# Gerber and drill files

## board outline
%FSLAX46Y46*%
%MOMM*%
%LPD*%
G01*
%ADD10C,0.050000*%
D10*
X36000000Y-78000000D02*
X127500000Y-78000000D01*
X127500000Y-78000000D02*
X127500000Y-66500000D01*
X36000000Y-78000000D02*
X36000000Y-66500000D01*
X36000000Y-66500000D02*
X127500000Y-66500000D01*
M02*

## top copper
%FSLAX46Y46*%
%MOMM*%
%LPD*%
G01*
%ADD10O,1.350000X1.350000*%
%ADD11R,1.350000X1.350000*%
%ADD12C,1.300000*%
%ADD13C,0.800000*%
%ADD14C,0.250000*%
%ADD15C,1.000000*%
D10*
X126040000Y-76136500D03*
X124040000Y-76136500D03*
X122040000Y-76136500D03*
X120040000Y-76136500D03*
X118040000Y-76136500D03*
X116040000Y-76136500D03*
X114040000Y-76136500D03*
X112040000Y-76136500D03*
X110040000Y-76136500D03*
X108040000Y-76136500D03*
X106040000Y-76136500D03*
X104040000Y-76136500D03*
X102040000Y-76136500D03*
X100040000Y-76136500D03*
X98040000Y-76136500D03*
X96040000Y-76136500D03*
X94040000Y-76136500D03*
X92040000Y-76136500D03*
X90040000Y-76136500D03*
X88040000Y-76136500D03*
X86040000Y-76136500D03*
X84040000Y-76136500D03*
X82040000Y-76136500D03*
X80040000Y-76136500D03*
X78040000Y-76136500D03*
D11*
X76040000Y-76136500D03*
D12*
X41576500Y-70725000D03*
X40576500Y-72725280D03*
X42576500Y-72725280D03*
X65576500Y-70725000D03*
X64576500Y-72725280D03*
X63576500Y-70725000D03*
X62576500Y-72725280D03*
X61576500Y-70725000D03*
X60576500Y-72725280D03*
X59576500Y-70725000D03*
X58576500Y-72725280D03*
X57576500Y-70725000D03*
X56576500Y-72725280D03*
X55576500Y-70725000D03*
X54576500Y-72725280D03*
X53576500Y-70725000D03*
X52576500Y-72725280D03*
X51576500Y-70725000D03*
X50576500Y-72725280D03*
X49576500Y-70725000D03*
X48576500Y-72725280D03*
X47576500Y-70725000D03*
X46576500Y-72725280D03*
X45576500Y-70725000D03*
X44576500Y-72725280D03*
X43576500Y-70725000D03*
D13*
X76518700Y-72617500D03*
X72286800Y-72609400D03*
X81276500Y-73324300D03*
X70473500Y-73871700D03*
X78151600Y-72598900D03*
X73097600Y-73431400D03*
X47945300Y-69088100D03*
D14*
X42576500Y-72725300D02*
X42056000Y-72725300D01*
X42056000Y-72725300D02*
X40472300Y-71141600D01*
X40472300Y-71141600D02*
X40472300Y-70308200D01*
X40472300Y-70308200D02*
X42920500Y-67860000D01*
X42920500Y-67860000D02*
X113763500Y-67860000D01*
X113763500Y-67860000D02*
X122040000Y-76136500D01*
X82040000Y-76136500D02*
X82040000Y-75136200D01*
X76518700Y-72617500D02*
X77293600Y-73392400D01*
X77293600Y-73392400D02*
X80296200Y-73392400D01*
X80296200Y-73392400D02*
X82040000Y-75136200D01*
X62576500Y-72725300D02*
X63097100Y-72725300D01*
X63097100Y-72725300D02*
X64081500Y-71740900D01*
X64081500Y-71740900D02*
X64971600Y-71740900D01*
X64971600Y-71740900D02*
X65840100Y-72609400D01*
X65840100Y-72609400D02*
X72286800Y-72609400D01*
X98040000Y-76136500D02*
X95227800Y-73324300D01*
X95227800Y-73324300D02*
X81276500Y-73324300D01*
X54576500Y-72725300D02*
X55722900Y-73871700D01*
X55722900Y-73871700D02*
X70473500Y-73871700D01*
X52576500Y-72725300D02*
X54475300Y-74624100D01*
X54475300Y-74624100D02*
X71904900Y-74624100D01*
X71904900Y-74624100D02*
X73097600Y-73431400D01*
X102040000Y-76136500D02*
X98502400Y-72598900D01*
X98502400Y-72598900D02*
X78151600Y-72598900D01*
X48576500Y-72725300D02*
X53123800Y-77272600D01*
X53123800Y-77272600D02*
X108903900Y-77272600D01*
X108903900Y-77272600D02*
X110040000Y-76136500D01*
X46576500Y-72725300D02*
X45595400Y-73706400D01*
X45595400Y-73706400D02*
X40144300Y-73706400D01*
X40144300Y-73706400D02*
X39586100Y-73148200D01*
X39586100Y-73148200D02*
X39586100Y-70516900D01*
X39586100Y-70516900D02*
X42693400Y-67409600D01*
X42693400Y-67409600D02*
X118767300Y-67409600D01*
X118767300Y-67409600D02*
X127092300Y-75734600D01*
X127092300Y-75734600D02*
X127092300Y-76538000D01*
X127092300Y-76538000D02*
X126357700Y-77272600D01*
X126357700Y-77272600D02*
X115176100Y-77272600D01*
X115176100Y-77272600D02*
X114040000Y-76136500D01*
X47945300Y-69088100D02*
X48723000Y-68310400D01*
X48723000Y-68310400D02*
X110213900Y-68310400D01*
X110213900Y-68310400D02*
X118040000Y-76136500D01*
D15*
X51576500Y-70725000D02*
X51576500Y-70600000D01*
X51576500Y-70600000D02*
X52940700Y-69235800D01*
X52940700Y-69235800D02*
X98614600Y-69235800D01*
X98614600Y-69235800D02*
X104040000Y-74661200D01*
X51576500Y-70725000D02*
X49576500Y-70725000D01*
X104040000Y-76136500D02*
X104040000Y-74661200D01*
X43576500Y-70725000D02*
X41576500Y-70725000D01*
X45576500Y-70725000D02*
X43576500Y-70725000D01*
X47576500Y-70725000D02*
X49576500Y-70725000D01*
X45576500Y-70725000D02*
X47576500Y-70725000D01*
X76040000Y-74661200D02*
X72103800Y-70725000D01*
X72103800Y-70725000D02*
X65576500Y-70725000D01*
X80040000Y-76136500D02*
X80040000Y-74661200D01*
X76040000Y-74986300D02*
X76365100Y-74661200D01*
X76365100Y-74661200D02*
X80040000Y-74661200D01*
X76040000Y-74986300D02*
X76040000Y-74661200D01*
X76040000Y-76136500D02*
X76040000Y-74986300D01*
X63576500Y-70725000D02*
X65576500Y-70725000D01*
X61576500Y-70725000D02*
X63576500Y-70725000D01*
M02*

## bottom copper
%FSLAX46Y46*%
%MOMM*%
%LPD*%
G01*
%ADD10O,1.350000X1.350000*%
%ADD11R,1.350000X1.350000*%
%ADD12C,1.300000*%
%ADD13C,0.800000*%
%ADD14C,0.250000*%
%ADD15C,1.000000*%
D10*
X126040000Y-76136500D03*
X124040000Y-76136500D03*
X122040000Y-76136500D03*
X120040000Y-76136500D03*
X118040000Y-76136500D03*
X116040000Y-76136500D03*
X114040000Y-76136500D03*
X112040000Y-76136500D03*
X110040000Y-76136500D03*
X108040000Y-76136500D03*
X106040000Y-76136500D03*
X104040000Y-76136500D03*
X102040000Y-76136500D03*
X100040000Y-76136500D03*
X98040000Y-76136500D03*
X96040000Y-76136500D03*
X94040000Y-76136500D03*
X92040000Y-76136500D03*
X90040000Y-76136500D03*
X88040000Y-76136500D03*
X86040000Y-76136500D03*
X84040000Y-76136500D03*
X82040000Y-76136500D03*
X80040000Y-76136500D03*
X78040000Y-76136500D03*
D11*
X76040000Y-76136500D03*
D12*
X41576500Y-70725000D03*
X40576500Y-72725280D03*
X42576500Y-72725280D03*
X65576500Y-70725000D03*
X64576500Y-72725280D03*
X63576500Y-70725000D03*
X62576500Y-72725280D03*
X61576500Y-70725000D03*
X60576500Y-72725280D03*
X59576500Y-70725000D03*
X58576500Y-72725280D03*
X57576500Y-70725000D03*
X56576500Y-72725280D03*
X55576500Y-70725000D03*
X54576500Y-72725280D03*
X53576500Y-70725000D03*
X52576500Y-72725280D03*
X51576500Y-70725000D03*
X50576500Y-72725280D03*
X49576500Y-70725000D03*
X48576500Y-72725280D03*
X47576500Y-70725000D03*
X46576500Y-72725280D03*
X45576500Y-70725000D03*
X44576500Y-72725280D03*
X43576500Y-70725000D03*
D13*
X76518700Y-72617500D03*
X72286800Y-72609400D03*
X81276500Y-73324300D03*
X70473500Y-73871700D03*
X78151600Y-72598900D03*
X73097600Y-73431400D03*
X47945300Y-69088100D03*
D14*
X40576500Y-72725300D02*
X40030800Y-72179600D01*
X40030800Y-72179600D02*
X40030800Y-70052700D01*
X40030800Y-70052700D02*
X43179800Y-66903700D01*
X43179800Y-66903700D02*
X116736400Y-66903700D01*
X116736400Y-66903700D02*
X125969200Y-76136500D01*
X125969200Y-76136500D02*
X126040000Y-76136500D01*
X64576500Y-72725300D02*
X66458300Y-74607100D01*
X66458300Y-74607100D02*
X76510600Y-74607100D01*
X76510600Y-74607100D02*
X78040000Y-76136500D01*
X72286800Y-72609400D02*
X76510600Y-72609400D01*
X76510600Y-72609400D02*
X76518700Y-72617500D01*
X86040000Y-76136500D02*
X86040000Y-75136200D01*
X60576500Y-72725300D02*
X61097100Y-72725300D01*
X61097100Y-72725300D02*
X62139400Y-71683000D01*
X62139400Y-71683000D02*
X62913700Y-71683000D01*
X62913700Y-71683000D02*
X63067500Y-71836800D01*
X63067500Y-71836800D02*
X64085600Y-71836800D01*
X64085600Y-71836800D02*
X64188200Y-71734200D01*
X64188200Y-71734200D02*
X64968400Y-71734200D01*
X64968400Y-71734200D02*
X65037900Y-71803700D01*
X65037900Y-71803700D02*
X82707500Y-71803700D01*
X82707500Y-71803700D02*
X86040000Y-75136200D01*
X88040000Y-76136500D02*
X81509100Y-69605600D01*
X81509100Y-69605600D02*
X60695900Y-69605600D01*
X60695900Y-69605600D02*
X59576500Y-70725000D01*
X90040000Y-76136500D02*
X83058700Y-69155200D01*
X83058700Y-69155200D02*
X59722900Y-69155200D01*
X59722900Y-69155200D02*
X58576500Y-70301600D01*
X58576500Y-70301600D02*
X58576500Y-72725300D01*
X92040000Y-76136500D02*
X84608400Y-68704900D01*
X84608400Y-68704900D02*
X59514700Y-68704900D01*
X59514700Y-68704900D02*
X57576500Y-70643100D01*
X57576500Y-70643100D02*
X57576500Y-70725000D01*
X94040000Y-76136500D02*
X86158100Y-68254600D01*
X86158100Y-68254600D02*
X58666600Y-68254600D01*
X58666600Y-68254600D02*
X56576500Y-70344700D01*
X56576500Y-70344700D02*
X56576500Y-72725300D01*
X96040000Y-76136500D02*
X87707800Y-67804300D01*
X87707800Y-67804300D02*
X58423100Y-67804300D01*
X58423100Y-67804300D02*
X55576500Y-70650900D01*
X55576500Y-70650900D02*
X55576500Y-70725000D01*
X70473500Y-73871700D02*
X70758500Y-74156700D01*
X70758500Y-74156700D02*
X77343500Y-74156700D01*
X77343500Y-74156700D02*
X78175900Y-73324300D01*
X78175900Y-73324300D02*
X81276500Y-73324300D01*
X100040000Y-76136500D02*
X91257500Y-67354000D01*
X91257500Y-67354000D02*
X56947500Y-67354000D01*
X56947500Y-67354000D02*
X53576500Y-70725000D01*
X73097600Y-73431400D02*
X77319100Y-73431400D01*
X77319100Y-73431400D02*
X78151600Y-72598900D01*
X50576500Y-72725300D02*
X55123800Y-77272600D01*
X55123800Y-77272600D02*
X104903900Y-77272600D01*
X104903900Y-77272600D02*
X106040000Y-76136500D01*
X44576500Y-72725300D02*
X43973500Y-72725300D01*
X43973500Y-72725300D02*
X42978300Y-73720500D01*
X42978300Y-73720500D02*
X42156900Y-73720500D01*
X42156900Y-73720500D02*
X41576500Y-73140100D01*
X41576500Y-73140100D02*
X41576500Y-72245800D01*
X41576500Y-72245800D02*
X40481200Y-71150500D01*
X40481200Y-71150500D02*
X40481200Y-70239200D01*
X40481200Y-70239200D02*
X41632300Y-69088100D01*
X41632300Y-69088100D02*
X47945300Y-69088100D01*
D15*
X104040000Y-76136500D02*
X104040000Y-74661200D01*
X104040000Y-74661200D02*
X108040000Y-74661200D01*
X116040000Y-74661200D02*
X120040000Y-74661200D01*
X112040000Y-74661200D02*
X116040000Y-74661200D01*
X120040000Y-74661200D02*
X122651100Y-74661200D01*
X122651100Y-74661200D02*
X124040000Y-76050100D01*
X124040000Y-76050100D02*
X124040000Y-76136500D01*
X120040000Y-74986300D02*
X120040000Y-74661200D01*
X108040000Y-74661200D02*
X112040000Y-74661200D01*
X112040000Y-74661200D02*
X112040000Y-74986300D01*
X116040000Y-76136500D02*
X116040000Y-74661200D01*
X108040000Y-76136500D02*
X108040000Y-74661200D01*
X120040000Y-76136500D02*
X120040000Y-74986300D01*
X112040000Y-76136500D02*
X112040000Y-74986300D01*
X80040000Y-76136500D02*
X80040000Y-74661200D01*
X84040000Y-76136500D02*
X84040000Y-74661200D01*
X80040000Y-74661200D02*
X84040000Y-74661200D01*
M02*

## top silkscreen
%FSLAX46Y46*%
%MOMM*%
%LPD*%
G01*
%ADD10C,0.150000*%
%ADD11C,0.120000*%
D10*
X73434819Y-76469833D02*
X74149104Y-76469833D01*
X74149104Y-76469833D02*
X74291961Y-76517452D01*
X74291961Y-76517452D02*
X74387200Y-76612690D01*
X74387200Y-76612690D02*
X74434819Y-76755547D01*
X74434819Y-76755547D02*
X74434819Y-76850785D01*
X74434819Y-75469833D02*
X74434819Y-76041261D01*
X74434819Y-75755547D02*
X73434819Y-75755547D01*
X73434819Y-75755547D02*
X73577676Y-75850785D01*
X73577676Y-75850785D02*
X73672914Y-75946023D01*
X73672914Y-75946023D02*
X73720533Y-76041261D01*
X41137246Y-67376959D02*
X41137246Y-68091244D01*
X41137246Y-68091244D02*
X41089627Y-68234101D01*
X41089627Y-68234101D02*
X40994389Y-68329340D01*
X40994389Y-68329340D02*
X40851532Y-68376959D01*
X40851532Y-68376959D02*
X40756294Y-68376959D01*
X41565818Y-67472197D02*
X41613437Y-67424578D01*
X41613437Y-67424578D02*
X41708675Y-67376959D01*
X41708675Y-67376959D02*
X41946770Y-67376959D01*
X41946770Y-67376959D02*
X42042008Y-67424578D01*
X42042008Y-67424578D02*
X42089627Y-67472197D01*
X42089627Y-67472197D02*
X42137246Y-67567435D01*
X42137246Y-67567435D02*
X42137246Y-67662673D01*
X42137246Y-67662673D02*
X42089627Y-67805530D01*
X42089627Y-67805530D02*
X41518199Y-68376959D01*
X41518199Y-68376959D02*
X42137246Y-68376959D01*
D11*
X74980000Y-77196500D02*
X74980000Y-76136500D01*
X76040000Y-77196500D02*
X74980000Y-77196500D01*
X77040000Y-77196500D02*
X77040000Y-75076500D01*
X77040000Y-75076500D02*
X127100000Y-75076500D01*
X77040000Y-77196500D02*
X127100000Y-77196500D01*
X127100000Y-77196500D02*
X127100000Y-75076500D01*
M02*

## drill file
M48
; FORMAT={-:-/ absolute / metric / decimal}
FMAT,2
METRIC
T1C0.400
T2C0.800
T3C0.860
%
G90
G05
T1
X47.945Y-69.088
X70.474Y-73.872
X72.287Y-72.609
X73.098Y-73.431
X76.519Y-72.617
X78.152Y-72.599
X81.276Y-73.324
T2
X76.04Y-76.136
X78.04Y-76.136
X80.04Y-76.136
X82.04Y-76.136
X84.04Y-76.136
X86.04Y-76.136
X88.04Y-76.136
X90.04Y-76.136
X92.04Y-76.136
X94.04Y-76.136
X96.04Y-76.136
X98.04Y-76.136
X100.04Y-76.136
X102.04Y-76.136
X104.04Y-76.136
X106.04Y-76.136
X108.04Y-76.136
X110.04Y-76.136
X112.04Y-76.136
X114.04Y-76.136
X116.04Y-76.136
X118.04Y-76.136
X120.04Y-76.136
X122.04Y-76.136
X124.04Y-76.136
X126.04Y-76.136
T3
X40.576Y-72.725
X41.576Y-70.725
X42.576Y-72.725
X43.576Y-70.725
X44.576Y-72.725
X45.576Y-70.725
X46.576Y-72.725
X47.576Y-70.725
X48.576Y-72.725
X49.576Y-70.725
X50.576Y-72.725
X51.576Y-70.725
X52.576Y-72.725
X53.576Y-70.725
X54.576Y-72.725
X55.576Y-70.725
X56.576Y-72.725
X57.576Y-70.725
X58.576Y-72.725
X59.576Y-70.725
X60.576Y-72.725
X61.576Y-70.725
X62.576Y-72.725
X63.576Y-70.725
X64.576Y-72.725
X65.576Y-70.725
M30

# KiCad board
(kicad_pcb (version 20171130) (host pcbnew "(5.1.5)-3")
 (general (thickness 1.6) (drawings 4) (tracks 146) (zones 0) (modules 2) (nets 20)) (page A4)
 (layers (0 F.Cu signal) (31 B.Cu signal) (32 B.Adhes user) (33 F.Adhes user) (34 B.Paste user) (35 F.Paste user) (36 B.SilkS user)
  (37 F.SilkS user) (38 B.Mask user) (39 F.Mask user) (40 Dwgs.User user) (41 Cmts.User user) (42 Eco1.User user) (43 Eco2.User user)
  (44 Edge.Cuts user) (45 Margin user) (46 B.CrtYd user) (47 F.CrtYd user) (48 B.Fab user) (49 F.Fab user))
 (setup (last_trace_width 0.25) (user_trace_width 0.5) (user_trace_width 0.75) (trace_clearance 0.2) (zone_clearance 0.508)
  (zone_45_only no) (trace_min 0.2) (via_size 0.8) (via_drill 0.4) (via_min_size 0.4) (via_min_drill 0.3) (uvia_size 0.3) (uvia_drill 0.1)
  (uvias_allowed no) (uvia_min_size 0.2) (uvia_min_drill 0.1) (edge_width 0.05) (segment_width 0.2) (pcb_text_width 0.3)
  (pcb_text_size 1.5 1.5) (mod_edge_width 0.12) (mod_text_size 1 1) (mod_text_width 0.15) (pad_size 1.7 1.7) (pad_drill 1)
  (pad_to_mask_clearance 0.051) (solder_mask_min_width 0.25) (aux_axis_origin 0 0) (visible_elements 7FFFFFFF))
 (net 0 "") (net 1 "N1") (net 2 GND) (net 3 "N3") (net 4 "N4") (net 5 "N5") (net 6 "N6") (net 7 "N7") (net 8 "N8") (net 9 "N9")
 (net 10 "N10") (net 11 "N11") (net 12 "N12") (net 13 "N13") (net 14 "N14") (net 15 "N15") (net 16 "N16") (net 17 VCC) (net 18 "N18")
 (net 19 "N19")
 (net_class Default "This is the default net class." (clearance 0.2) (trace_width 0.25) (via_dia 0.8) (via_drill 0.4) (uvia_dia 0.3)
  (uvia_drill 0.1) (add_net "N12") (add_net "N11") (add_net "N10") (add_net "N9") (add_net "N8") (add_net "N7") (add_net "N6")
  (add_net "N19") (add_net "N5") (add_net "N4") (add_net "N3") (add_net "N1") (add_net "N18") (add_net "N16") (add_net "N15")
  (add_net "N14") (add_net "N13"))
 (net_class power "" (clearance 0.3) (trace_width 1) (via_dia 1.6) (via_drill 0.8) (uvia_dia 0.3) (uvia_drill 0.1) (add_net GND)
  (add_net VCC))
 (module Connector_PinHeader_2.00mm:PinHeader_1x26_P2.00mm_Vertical (layer F.Cu) (at 76.04 76.1365 90)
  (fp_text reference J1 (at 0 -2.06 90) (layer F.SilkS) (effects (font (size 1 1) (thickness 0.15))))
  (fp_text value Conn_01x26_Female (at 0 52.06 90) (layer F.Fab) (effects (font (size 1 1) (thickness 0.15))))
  (fp_line (start -1.06 -1.06) (end 0 -1.06) (layer F.SilkS) (width 0.12))
  (fp_line (start -1.06 0) (end -1.06 -1.06) (layer F.SilkS) (width 0.12))
  (fp_line (start -1.06 1) (end 1.06 1) (layer F.SilkS) (width 0.12))
  (fp_line (start 1.06 1) (end 1.06 51.06) (layer F.SilkS) (width 0.12))
  (fp_line (start -1.06 1) (end -1.06 51.06) (layer F.SilkS) (width 0.12))
  (fp_line (start -1.06 51.06) (end 1.06 51.06) (layer F.SilkS) (width 0.12))
  (pad 26 thru_hole oval (at 0 50 90) (size 1.35 1.35) (drill 0.8) (layers *.Cu *.Mask) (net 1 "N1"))
  (pad 25 thru_hole oval (at 0 48 90) (size 1.35 1.35) (drill 0.8) (layers *.Cu *.Mask) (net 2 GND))
  (pad 24 thru_hole oval (at 0 46 90) (size 1.35 1.35) (drill 0.8) (layers *.Cu *.Mask) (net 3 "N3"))
  (pad 23 thru_hole oval (at 0 44 90) (size 1.35 1.35) (drill 0.8) (layers *.Cu *.Mask) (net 2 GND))
  (pad 22 thru_hole oval (at 0 42 90) (size 1.35 1.35) (drill 0.8) (layers *.Cu *.Mask) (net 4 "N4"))
  (pad 21 thru_hole oval (at 0 40 90) (size 1.35 1.35) (drill 0.8) (layers *.Cu *.Mask) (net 2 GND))
  (pad 20 thru_hole oval (at 0 38 90) (size 1.35 1.35) (drill 0.8) (layers *.Cu *.Mask) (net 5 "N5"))
  (pad 19 thru_hole oval (at 0 36 90) (size 1.35 1.35) (drill 0.8) (layers *.Cu *.Mask) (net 2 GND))
  (pad 18 thru_hole oval (at 0 34 90) (size 1.35 1.35) (drill 0.8) (layers *.Cu *.Mask) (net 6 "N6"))
  (pad 17 thru_hole oval (at 0 32 90) (size 1.35 1.35) (drill 0.8) (layers *.Cu *.Mask) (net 2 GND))
  (pad 16 thru_hole oval (at 0 30 90) (size 1.35 1.35) (drill 0.8) (layers *.Cu *.Mask) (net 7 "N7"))
  (pad 15 thru_hole oval (at 0 28 90) (size 1.35 1.35) (drill 0.8) (layers *.Cu *.Mask) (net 2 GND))
  (pad 14 thru_hole oval (at 0 26 90) (size 1.35 1.35) (drill 0.8) (layers *.Cu *.Mask) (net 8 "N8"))
  (pad 13 thru_hole oval (at 0 24 90) (size 1.35 1.35) (drill 0.8) (layers *.Cu *.Mask) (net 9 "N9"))
  (pad 12 thru_hole oval (at 0 22 90) (size 1.35 1.35) (drill 0.8) (layers *.Cu *.Mask) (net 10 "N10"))
  (pad 11 thru_hole oval (at 0 20 90) (size 1.35 1.35) (drill 0.8) (layers *.Cu *.Mask) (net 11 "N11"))
  (pad 10 thru_hole oval (at 0 18 90) (size 1.35 1.35) (drill 0.8) (layers *.Cu *.Mask) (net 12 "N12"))
  (pad 9 thru_hole oval (at 0 16 90) (size 1.35 1.35) (drill 0.8) (layers *.Cu *.Mask) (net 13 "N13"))
  (pad 8 thru_hole oval (at 0 14 90) (size 1.35 1.35) (drill 0.8) (layers *.Cu *.Mask) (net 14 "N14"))
  (pad 7 thru_hole oval (at 0 12 90) (size 1.35 1.35) (drill 0.8) (layers *.Cu *.Mask) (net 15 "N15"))
  (pad 6 thru_hole oval (at 0 10 90) (size 1.35 1.35) (drill 0.8) (layers *.Cu *.Mask) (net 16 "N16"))
  (pad 5 thru_hole oval (at 0 8 90) (size 1.35 1.35) (drill 0.8) (layers *.Cu *.Mask) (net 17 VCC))
  (pad 4 thru_hole oval (at 0 6 90) (size 1.35 1.35) (drill 0.8) (layers *.Cu *.Mask) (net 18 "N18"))
  (pad 3 thru_hole oval (at 0 4 90) (size 1.35 1.35) (drill 0.8) (layers *.Cu *.Mask) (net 17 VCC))
  (pad 2 thru_hole oval (at 0 2 90) (size 1.35 1.35) (drill 0.8) (layers *.Cu *.Mask) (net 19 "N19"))
  (pad 1 thru_hole rect (at 0 0 90) (size 1.35 1.35) (drill 0.8) (layers *.Cu *.Mask) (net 17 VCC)))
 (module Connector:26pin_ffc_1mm (layer F.Cu) (at 40.5765 75.438)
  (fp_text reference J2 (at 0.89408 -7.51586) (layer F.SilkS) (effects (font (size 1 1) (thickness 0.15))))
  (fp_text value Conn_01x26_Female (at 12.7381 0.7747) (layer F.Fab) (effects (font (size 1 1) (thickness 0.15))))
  (pad 25 thru_hole circle (at 1 -4.713) (size 1.3 1.3) (drill 0.86) (layers *.Cu *.Mask) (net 2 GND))
  (pad 26 thru_hole circle (at 0 -2.71272) (size 1.3 1.3) (drill 0.86) (layers *.Cu *.Mask) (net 1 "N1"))
  (pad 24 thru_hole circle (at 2 -2.71272) (size 1.3 1.3) (drill 0.86) (layers *.Cu *.Mask) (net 3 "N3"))
  (pad 1 thru_hole circle (at 25 -4.713) (size 1.3 1.3) (drill 0.86) (layers *.Cu *.Mask) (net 17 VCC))
  (pad 2 thru_hole circle (at 24 -2.71272) (size 1.3 1.3) (drill 0.86) (layers *.Cu *.Mask) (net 19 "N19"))
  (pad 3 thru_hole circle (at 23 -4.713) (size 1.3 1.3) (drill 0.86) (layers *.Cu *.Mask) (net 17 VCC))
  (pad 4 thru_hole circle (at 22 -2.71272) (size 1.3 1.3) (drill 0.86) (layers *.Cu *.Mask) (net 18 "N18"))
  (pad 5 thru_hole circle (at 21 -4.713) (size 1.3 1.3) (drill 0.86) (layers *.Cu *.Mask) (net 17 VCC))
  (pad 6 thru_hole circle (at 20 -2.71272) (size 1.3 1.3) (drill 0.86) (layers *.Cu *.Mask) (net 16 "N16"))
  (pad 7 thru_hole circle (at 19 -4.713) (size 1.3 1.3) (drill 0.86) (layers *.Cu *.Mask) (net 15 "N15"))
  (pad 8 thru_hole circle (at 18 -2.71272) (size 1.3 1.3) (drill 0.86) (layers *.Cu *.Mask) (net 14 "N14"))
  (pad 9 thru_hole circle (at 17 -4.713) (size 1.3 1.3) (drill 0.86) (layers *.Cu *.Mask) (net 13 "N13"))
  (pad 10 thru_hole circle (at 16 -2.71272) (size 1.3 1.3) (drill 0.86) (layers *.Cu *.Mask) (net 12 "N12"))
  (pad 11 thru_hole circle (at 15 -4.713) (size 1.3 1.3) (drill 0.86) (layers *.Cu *.Mask) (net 11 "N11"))
  (pad 12 thru_hole circle (at 14 -2.71272) (size 1.3 1.3) (drill 0.86) (layers *.Cu *.Mask) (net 10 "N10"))
  (pad 13 thru_hole circle (at 13 -4.713) (size 1.3 1.3) (drill 0.86) (layers *.Cu *.Mask) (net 9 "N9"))
  (pad 14 thru_hole circle (at 12 -2.71272) (size 1.3 1.3) (drill 0.86) (layers *.Cu *.Mask) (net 8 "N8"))
  (pad 15 thru_hole circle (at 11 -4.713) (size 1.3 1.3) (drill 0.86) (layers *.Cu *.Mask) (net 2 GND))
  (pad 16 thru_hole circle (at 10 -2.71272) (size 1.3 1.3) (drill 0.86) (layers *.Cu *.Mask) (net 7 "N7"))
  (pad 17 thru_hole circle (at 9 -4.713) (size 1.3 1.3) (drill 0.86) (layers *.Cu *.Mask) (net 2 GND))
  (pad 18 thru_hole circle (at 8 -2.71272) (size 1.3 1.3) (drill 0.86) (layers *.Cu *.Mask) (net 6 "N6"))
  (pad 19 thru_hole circle (at 7 -4.713) (size 1.3 1.3) (drill 0.86) (layers *.Cu *.Mask) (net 2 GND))
  (pad 20 thru_hole circle (at 6 -2.71272) (size 1.3 1.3) (drill 0.86) (layers *.Cu *.Mask) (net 5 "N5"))
  (pad 21 thru_hole circle (at 5 -4.713) (size 1.3 1.3) (drill 0.86) (layers *.Cu *.Mask) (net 2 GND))
  (pad 22 thru_hole circle (at 4 -2.71272) (size 1.3 1.3) (drill 0.86) (layers *.Cu *.Mask) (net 4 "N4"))
  (pad 23 thru_hole circle (at 3 -4.713) (size 1.3 1.3) (drill 0.86) (layers *.Cu *.Mask) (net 2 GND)))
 (gr_line (start 36 78) (end 127.5 78) (layer Edge.Cuts) (width 0.05))
 (gr_line (start 127.5 78) (end 127.5 66.5) (layer Edge.Cuts) (width 0.05))
 (gr_line (start 36 78) (end 36 66.5) (layer Edge.Cuts) (width 0.05))
 (gr_line (start 36 66.5) (end 127.5 66.5) (layer Edge.Cuts) (width 0.05))
 (segment (start 40.5765 72.7253) (end 40.0308 72.1796) (width 0.25) (layer B.Cu) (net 1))
 (segment (start 40.0308 72.1796) (end 40.0308 70.0527) (width 0.25) (layer B.Cu) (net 1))
 (segment (start 40.0308 70.0527) (end 43.1798 66.9037) (width 0.25) (layer B.Cu) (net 1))
 (segment (start 43.1798 66.9037) (end 116.7364 66.9037) (width 0.25) (layer B.Cu) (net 1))
 (segment (start 116.7364 66.9037) (end 125.9692 76.1365) (width 0.25) (layer B.Cu) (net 1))
 (segment (start 125.9692 76.1365) (end 126.04 76.1365) (width 0.25) (layer B.Cu) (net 1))
 (segment (start 42.5765 72.7253) (end 42.056 72.7253) (width 0.25) (layer F.Cu) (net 3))
 (segment (start 42.056 72.7253) (end 40.4723 71.1416) (width 0.25) (layer F.Cu) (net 3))
 (segment (start 40.4723 71.1416) (end 40.4723 70.3082) (width 0.25) (layer F.Cu) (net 3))
 (segment (start 40.4723 70.3082) (end 42.9205 67.86) (width 0.25) (layer F.Cu) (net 3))
 (segment (start 42.9205 67.86) (end 113.7635 67.86) (width 0.25) (layer F.Cu) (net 3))
 (segment (start 113.7635 67.86) (end 122.04 76.1365) (width 0.25) (layer F.Cu) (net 3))
 (segment (start 64.5765 72.7253) (end 66.4583 74.6071) (width 0.25) (layer B.Cu) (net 19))
 (segment (start 66.4583 74.6071) (end 76.5106 74.6071) (width 0.25) (layer B.Cu) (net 19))
 (segment (start 76.5106 74.6071) (end 78.04 76.1365) (width 0.25) (layer B.Cu) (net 19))
 (segment (start 82.04 76.1365) (end 82.04 75.1362) (width 0.25) (layer F.Cu) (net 18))
 (segment (start 76.5187 72.6175) (end 77.2936 73.3924) (width 0.25) (layer F.Cu) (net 18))
 (segment (start 77.2936 73.3924) (end 80.2962 73.3924) (width 0.25) (layer F.Cu) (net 18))
 (segment (start 80.2962 73.3924) (end 82.04 75.1362) (width 0.25) (layer F.Cu) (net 18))
 (segment (start 72.2868 72.6094) (end 76.5106 72.6094) (width 0.25) (layer B.Cu) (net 18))
 (segment (start 76.5106 72.6094) (end 76.5187 72.6175) (width 0.25) (layer B.Cu) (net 18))
 (segment (start 62.5765 72.7253) (end 63.0971 72.7253) (width 0.25) (layer F.Cu) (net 18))
 (segment (start 63.0971 72.7253) (end 64.0815 71.7409) (width 0.25) (layer F.Cu) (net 18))
 (segment (start 64.0815 71.7409) (end 64.9716 71.7409) (width 0.25) (layer F.Cu) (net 18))
 (segment (start 64.9716 71.7409) (end 65.8401 72.6094) (width 0.25) (layer F.Cu) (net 18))
 (segment (start 65.8401 72.6094) (end 72.2868 72.6094) (width 0.25) (layer F.Cu) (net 18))
 (via (at 76.5187 72.6175) (size 0.8) (layers F.Cu B.Cu) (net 18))
 (via (at 72.2868 72.6094) (size 0.8) (layers F.Cu B.Cu) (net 18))
 (segment (start 86.04 76.1365) (end 86.04 75.1362) (width 0.25) (layer B.Cu) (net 16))
 (segment (start 60.5765 72.7253) (end 61.0971 72.7253) (width 0.25) (layer B.Cu) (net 16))
 (segment (start 61.0971 72.7253) (end 62.1394 71.683) (width 0.25) (layer B.Cu) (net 16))
 (segment (start 62.1394 71.683) (end 62.9137 71.683) (width 0.25) (layer B.Cu) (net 16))
 (segment (start 62.9137 71.683) (end 63.0675 71.8368) (width 0.25) (layer B.Cu) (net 16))
 (segment (start 63.0675 71.8368) (end 64.0856 71.8368) (width 0.25) (layer B.Cu) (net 16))
 (segment (start 64.0856 71.8368) (end 64.1882 71.7342) (width 0.25) (layer B.Cu) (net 16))
 (segment (start 64.1882 71.7342) (end 64.9684 71.7342) (width 0.25) (layer B.Cu) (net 16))
 (segment (start 64.9684 71.7342) (end 65.0379 71.8037) (width 0.25) (layer B.Cu) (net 16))
 (segment (start 65.0379 71.8037) (end 82.7075 71.8037) (width 0.25) (layer B.Cu) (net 16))
 (segment (start 82.7075 71.8037) (end 86.04 75.1362) (width 0.25) (layer B.Cu) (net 16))
 (segment (start 88.04 76.1365) (end 81.5091 69.6056) (width 0.25) (layer B.Cu) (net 15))
 (segment (start 81.5091 69.6056) (end 60.6959 69.6056) (width 0.25) (layer B.Cu) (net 15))
 (segment (start 60.6959 69.6056) (end 59.5765 70.725) (width 0.25) (layer B.Cu) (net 15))
 (segment (start 90.04 76.1365) (end 83.0587 69.1552) (width 0.25) (layer B.Cu) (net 14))
 (segment (start 83.0587 69.1552) (end 59.7229 69.1552) (width 0.25) (layer B.Cu) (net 14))
 (segment (start 59.7229 69.1552) (end 58.5765 70.3016) (width 0.25) (layer B.Cu) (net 14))
 (segment (start 58.5765 70.3016) (end 58.5765 72.7253) (width 0.25) (layer B.Cu) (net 14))
 (segment (start 92.04 76.1365) (end 84.6084 68.7049) (width 0.25) (layer B.Cu) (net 13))
 (segment (start 84.6084 68.7049) (end 59.5147 68.7049) (width 0.25) (layer B.Cu) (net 13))
 (segment (start 59.5147 68.7049) (end 57.5765 70.6431) (width 0.25) (layer B.Cu) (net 13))
 (segment (start 57.5765 70.6431) (end 57.5765 70.725) (width 0.25) (layer B.Cu) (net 13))
 (segment (start 94.04 76.1365) (end 86.1581 68.2546) (width 0.25) (layer B.Cu) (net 12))
 (segment (start 86.1581 68.2546) (end 58.6666 68.2546) (width 0.25) (layer B.Cu) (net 12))
 (segment (start 58.6666 68.2546) (end 56.5765 70.3447) (width 0.25) (layer B.Cu) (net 12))
 (segment (start 56.5765 70.3447) (end 56.5765 72.7253) (width 0.25) (layer B.Cu) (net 12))
 (segment (start 96.04 76.1365) (end 87.7078 67.8043) (width 0.25) (layer B.Cu) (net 11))
 (segment (start 87.7078 67.8043) (end 58.4231 67.8043) (width 0.25) (layer B.Cu) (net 11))
 (segment (start 58.4231 67.8043) (end 55.5765 70.6509) (width 0.25) (layer B.Cu) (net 11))
 (segment (start 55.5765 70.6509) (end 55.5765 70.725) (width 0.25) (layer B.Cu) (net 11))
 (segment (start 98.04 76.1365) (end 95.2278 73.3243) (width 0.25) (layer F.Cu) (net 10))
 (segment (start 95.2278 73.3243) (end 81.2765 73.3243) (width 0.25) (layer F.Cu) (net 10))
 (segment (start 70.4735 73.8717) (end 70.7585 74.1567) (width 0.25) (layer B.Cu) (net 10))
 (segment (start 70.7585 74.1567) (end 77.3435 74.1567) (width 0.25) (layer B.Cu) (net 10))
 (segment (start 77.3435 74.1567) (end 78.1759 73.3243) (width 0.25) (layer B.Cu) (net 10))
 (segment (start 78.1759 73.3243) (end 81.2765 73.3243) (width 0.25) (layer B.Cu) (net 10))
 (segment (start 54.5765 72.7253) (end 55.7229 73.8717) (width 0.25) (layer F.Cu) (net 10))
 (segment (start 55.7229 73.8717) (end 70.4735 73.8717) (width 0.25) (layer F.Cu) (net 10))
 (via (at 81.2765 73.3243) (size 0.8) (layers F.Cu B.Cu) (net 10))
 (via (at 70.4735 73.8717) (size 0.8) (layers F.Cu B.Cu) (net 10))
 (segment (start 100.04 76.1365) (end 91.2575 67.354) (width 0.25) (layer B.Cu) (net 9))
 (segment (start 91.2575 67.354) (end 56.9475 67.354) (width 0.25) (layer B.Cu) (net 9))
 (segment (start 56.9475 67.354) (end 53.5765 70.725) (width 0.25) (layer B.Cu) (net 9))
 (segment (start 52.5765 72.7253) (end 54.4753 74.6241) (width 0.25) (layer F.Cu) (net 8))
 (segment (start 54.4753 74.6241) (end 71.9049 74.6241) (width 0.25) (layer F.Cu) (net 8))
 (segment (start 71.9049 74.6241) (end 73.0976 73.4314) (width 0.25) (layer F.Cu) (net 8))
 (segment (start 73.0976 73.4314) (end 77.3191 73.4314) (width 0.25) (layer B.Cu) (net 8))
 (segment (start 77.3191 73.4314) (end 78.1516 72.5989) (width 0.25) (layer B.Cu) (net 8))
 (segment (start 102.04 76.1365) (end 98.5024 72.5989) (width 0.25) (layer F.Cu) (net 8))
 (segment (start 98.5024 72.5989) (end 78.1516 72.5989) (width 0.25) (layer F.Cu) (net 8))
 (via (at 78.1516 72.5989) (size 0.8) (layers F.Cu B.Cu) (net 8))
 (via (at 73.0976 73.4314) (size 0.8) (layers F.Cu B.Cu) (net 8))
 (segment (start 50.5765 72.7253) (end 55.1238 77.2726) (width 0.25) (layer B.Cu) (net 7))
 (segment (start 55.1238 77.2726) (end 104.9039 77.2726) (width 0.25) (layer B.Cu) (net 7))
 (segment (start 104.9039 77.2726) (end 106.04 76.1365) (width 0.25) (layer B.Cu) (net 7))
 (segment (start 48.5765 72.7253) (end 53.1238 77.2726) (width 0.25) (layer F.Cu) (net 6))
 (segment (start 53.1238 77.2726) (end 108.9039 77.2726) (width 0.25) (layer F.Cu) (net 6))
 (segment (start 108.9039 77.2726) (end 110.04 76.1365) (width 0.25) (layer F.Cu) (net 6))
 (segment (start 46.5765 72.7253) (end 45.5954 73.7064) (width 0.25) (layer F.Cu) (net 5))
 (segment (start 45.5954 73.7064) (end 40.1443 73.7064) (width 0.25) (layer F.Cu) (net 5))
 (segment (start 40.1443 73.7064) (end 39.5861 73.1482) (width 0.25) (layer F.Cu) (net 5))
 (segment (start 39.5861 73.1482) (end 39.5861 70.5169) (width 0.25) (layer F.Cu) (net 5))
 (segment (start 39.5861 70.5169) (end 42.6934 67.4096) (width 0.25) (layer F.Cu) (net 5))
 (segment (start 42.6934 67.4096) (end 118.7673 67.4096) (width 0.25) (layer F.Cu) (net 5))
 (segment (start 118.7673 67.4096) (end 127.0923 75.7346) (width 0.25) (layer F.Cu) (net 5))
 (segment (start 127.0923 75.7346) (end 127.0923 76.538) (width 0.25) (layer F.Cu) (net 5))
 (segment (start 127.0923 76.538) (end 126.3577 77.2726) (width 0.25) (layer F.Cu) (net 5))
 (segment (start 126.3577 77.2726) (end 115.1761 77.2726) (width 0.25) (layer F.Cu) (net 5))
 (segment (start 115.1761 77.2726) (end 114.04 76.1365) (width 0.25) (layer F.Cu) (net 5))
 (segment (start 44.5765 72.7253) (end 43.9735 72.7253) (width 0.25) (layer B.Cu) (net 4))
 (segment (start 43.9735 72.7253) (end 42.9783 73.7205) (width 0.25) (layer B.Cu) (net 4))
 (segment (start 42.9783 73.7205) (end 42.1569 73.7205) (width 0.25) (layer B.Cu) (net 4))
 (segment (start 42.1569 73.7205) (end 41.5765 73.1401) (width 0.25) (layer B.Cu) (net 4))
 (segment (start 41.5765 73.1401) (end 41.5765 72.2458) (width 0.25) (layer B.Cu) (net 4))
 (segment (start 41.5765 72.2458) (end 40.4812 71.1505) (width 0.25) (layer B.Cu) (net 4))
 (segment (start 40.4812 71.1505) (end 40.4812 70.2392) (width 0.25) (layer B.Cu) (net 4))
 (segment (start 40.4812 70.2392) (end 41.6323 69.0881) (width 0.25) (layer B.Cu) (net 4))
 (segment (start 41.6323 69.0881) (end 47.9453 69.0881) (width 0.25) (layer B.Cu) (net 4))
 (segment (start 47.9453 69.0881) (end 48.723 68.3104) (width 0.25) (layer F.Cu) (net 4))
 (segment (start 48.723 68.3104) (end 110.2139 68.3104) (width 0.25) (layer F.Cu) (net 4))
 (segment (start 110.2139 68.3104) (end 118.04 76.1365) (width 0.25) (layer F.Cu) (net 4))
 (via (at 47.9453 69.0881) (size 0.8) (layers F.Cu B.Cu) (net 4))
 (segment (start 104.04 76.1365) (end 104.04 74.6612) (width 1) (layer B.Cu) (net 2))
 (segment (start 104.04 74.6612) (end 108.04 74.6612) (width 1) (layer B.Cu) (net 2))
 (segment (start 51.5765 70.725) (end 51.5765 70.6) (width 1) (layer F.Cu) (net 2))
 (segment (start 51.5765 70.6) (end 52.9407 69.2358) (width 1) (layer F.Cu) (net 2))
 (segment (start 52.9407 69.2358) (end 98.6146 69.2358) (width 1) (layer F.Cu) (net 2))
 (segment (start 98.6146 69.2358) (end 104.04 74.6612) (width 1) (layer F.Cu) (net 2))
 (segment (start 51.5765 70.725) (end 49.5765 70.725) (width 1) (layer F.Cu) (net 2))
 (segment (start 104.04 76.1365) (end 104.04 74.6612) (width 1) (layer F.Cu) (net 2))
 (segment (start 116.04 74.6612) (end 120.04 74.6612) (width 1) (layer B.Cu) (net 2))
 (segment (start 112.04 74.6612) (end 116.04 74.6612) (width 1) (layer B.Cu) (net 2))
 (segment (start 120.04 74.6612) (end 122.6511 74.6612) (width 1) (layer B.Cu) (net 2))
 (segment (start 122.6511 74.6612) (end 124.04 76.0501) (width 1) (layer B.Cu) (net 2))
 (segment (start 124.04 76.0501) (end 124.04 76.1365) (width 1) (layer B.Cu) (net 2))
 (segment (start 120.04 74.9863) (end 120.04 74.6612) (width 1) (layer B.Cu) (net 2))
 (segment (start 108.04 74.6612) (end 112.04 74.6612) (width 1) (layer B.Cu) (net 2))
 (segment (start 112.04 74.6612) (end 112.04 74.9863) (width 1) (layer B.Cu) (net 2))
 (segment (start 116.04 76.1365) (end 116.04 74.6612) (width 1) (layer B.Cu) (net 2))
 (segment (start 108.04 76.1365) (end 108.04 74.6612) (width 1) (layer B.Cu) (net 2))
 (segment (start 120.04 76.1365) (end 120.04 74.9863) (width 1) (layer B.Cu) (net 2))
 (segment (start 112.04 76.1365) (end 112.04 74.9863) (width 1) (layer B.Cu) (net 2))
 (segment (start 43.5765 70.725) (end 41.5765 70.725) (width 1) (layer F.Cu) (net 2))
 (segment (start 45.5765 70.725) (end 43.5765 70.725) (width 1) (layer F.Cu) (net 2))
 (segment (start 47.5765 70.725) (end 49.5765 70.725) (width 1) (layer F.Cu) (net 2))
 (segment (start 45.5765 70.725) (end 47.5765 70.725) (width 1) (layer F.Cu) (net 2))
 (segment (start 76.04 74.6612) (end 72.1038 70.725) (width 1) (layer F.Cu) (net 17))
 (segment (start 72.1038 70.725) (end 65.5765 70.725) (width 1) (layer F.Cu) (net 17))
 (segment (start 80.04 76.1365) (end 80.04 74.6612) (width 1) (layer B.Cu) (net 17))
 (segment (start 80.04 76.1365) (end 80.04 74.6612) (width 1) (layer F.Cu) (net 17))
 (segment (start 76.04 74.9863) (end 76.3651 74.6612) (width 1) (layer F.Cu) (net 17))
 (segment (start 76.3651 74.6612) (end 80.04 74.6612) (width 1) (layer F.Cu) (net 17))
 (segment (start 76.04 74.9863) (end 76.04 74.6612) (width 1) (layer F.Cu) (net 17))
 (segment (start 76.04 76.1365) (end 76.04 74.9863) (width 1) (layer F.Cu) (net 17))
 (segment (start 63.5765 70.725) (end 65.5765 70.725) (width 1) (layer F.Cu) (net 17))
 (segment (start 84.04 76.1365) (end 84.04 74.6612) (width 1) (layer B.Cu) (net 17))
 (segment (start 80.04 74.6612) (end 84.04 74.6612) (width 1) (layer B.Cu) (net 17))
 (segment (start 61.5765 70.725) (end 63.5765 70.725) (width 1) (layer F.Cu) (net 17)))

